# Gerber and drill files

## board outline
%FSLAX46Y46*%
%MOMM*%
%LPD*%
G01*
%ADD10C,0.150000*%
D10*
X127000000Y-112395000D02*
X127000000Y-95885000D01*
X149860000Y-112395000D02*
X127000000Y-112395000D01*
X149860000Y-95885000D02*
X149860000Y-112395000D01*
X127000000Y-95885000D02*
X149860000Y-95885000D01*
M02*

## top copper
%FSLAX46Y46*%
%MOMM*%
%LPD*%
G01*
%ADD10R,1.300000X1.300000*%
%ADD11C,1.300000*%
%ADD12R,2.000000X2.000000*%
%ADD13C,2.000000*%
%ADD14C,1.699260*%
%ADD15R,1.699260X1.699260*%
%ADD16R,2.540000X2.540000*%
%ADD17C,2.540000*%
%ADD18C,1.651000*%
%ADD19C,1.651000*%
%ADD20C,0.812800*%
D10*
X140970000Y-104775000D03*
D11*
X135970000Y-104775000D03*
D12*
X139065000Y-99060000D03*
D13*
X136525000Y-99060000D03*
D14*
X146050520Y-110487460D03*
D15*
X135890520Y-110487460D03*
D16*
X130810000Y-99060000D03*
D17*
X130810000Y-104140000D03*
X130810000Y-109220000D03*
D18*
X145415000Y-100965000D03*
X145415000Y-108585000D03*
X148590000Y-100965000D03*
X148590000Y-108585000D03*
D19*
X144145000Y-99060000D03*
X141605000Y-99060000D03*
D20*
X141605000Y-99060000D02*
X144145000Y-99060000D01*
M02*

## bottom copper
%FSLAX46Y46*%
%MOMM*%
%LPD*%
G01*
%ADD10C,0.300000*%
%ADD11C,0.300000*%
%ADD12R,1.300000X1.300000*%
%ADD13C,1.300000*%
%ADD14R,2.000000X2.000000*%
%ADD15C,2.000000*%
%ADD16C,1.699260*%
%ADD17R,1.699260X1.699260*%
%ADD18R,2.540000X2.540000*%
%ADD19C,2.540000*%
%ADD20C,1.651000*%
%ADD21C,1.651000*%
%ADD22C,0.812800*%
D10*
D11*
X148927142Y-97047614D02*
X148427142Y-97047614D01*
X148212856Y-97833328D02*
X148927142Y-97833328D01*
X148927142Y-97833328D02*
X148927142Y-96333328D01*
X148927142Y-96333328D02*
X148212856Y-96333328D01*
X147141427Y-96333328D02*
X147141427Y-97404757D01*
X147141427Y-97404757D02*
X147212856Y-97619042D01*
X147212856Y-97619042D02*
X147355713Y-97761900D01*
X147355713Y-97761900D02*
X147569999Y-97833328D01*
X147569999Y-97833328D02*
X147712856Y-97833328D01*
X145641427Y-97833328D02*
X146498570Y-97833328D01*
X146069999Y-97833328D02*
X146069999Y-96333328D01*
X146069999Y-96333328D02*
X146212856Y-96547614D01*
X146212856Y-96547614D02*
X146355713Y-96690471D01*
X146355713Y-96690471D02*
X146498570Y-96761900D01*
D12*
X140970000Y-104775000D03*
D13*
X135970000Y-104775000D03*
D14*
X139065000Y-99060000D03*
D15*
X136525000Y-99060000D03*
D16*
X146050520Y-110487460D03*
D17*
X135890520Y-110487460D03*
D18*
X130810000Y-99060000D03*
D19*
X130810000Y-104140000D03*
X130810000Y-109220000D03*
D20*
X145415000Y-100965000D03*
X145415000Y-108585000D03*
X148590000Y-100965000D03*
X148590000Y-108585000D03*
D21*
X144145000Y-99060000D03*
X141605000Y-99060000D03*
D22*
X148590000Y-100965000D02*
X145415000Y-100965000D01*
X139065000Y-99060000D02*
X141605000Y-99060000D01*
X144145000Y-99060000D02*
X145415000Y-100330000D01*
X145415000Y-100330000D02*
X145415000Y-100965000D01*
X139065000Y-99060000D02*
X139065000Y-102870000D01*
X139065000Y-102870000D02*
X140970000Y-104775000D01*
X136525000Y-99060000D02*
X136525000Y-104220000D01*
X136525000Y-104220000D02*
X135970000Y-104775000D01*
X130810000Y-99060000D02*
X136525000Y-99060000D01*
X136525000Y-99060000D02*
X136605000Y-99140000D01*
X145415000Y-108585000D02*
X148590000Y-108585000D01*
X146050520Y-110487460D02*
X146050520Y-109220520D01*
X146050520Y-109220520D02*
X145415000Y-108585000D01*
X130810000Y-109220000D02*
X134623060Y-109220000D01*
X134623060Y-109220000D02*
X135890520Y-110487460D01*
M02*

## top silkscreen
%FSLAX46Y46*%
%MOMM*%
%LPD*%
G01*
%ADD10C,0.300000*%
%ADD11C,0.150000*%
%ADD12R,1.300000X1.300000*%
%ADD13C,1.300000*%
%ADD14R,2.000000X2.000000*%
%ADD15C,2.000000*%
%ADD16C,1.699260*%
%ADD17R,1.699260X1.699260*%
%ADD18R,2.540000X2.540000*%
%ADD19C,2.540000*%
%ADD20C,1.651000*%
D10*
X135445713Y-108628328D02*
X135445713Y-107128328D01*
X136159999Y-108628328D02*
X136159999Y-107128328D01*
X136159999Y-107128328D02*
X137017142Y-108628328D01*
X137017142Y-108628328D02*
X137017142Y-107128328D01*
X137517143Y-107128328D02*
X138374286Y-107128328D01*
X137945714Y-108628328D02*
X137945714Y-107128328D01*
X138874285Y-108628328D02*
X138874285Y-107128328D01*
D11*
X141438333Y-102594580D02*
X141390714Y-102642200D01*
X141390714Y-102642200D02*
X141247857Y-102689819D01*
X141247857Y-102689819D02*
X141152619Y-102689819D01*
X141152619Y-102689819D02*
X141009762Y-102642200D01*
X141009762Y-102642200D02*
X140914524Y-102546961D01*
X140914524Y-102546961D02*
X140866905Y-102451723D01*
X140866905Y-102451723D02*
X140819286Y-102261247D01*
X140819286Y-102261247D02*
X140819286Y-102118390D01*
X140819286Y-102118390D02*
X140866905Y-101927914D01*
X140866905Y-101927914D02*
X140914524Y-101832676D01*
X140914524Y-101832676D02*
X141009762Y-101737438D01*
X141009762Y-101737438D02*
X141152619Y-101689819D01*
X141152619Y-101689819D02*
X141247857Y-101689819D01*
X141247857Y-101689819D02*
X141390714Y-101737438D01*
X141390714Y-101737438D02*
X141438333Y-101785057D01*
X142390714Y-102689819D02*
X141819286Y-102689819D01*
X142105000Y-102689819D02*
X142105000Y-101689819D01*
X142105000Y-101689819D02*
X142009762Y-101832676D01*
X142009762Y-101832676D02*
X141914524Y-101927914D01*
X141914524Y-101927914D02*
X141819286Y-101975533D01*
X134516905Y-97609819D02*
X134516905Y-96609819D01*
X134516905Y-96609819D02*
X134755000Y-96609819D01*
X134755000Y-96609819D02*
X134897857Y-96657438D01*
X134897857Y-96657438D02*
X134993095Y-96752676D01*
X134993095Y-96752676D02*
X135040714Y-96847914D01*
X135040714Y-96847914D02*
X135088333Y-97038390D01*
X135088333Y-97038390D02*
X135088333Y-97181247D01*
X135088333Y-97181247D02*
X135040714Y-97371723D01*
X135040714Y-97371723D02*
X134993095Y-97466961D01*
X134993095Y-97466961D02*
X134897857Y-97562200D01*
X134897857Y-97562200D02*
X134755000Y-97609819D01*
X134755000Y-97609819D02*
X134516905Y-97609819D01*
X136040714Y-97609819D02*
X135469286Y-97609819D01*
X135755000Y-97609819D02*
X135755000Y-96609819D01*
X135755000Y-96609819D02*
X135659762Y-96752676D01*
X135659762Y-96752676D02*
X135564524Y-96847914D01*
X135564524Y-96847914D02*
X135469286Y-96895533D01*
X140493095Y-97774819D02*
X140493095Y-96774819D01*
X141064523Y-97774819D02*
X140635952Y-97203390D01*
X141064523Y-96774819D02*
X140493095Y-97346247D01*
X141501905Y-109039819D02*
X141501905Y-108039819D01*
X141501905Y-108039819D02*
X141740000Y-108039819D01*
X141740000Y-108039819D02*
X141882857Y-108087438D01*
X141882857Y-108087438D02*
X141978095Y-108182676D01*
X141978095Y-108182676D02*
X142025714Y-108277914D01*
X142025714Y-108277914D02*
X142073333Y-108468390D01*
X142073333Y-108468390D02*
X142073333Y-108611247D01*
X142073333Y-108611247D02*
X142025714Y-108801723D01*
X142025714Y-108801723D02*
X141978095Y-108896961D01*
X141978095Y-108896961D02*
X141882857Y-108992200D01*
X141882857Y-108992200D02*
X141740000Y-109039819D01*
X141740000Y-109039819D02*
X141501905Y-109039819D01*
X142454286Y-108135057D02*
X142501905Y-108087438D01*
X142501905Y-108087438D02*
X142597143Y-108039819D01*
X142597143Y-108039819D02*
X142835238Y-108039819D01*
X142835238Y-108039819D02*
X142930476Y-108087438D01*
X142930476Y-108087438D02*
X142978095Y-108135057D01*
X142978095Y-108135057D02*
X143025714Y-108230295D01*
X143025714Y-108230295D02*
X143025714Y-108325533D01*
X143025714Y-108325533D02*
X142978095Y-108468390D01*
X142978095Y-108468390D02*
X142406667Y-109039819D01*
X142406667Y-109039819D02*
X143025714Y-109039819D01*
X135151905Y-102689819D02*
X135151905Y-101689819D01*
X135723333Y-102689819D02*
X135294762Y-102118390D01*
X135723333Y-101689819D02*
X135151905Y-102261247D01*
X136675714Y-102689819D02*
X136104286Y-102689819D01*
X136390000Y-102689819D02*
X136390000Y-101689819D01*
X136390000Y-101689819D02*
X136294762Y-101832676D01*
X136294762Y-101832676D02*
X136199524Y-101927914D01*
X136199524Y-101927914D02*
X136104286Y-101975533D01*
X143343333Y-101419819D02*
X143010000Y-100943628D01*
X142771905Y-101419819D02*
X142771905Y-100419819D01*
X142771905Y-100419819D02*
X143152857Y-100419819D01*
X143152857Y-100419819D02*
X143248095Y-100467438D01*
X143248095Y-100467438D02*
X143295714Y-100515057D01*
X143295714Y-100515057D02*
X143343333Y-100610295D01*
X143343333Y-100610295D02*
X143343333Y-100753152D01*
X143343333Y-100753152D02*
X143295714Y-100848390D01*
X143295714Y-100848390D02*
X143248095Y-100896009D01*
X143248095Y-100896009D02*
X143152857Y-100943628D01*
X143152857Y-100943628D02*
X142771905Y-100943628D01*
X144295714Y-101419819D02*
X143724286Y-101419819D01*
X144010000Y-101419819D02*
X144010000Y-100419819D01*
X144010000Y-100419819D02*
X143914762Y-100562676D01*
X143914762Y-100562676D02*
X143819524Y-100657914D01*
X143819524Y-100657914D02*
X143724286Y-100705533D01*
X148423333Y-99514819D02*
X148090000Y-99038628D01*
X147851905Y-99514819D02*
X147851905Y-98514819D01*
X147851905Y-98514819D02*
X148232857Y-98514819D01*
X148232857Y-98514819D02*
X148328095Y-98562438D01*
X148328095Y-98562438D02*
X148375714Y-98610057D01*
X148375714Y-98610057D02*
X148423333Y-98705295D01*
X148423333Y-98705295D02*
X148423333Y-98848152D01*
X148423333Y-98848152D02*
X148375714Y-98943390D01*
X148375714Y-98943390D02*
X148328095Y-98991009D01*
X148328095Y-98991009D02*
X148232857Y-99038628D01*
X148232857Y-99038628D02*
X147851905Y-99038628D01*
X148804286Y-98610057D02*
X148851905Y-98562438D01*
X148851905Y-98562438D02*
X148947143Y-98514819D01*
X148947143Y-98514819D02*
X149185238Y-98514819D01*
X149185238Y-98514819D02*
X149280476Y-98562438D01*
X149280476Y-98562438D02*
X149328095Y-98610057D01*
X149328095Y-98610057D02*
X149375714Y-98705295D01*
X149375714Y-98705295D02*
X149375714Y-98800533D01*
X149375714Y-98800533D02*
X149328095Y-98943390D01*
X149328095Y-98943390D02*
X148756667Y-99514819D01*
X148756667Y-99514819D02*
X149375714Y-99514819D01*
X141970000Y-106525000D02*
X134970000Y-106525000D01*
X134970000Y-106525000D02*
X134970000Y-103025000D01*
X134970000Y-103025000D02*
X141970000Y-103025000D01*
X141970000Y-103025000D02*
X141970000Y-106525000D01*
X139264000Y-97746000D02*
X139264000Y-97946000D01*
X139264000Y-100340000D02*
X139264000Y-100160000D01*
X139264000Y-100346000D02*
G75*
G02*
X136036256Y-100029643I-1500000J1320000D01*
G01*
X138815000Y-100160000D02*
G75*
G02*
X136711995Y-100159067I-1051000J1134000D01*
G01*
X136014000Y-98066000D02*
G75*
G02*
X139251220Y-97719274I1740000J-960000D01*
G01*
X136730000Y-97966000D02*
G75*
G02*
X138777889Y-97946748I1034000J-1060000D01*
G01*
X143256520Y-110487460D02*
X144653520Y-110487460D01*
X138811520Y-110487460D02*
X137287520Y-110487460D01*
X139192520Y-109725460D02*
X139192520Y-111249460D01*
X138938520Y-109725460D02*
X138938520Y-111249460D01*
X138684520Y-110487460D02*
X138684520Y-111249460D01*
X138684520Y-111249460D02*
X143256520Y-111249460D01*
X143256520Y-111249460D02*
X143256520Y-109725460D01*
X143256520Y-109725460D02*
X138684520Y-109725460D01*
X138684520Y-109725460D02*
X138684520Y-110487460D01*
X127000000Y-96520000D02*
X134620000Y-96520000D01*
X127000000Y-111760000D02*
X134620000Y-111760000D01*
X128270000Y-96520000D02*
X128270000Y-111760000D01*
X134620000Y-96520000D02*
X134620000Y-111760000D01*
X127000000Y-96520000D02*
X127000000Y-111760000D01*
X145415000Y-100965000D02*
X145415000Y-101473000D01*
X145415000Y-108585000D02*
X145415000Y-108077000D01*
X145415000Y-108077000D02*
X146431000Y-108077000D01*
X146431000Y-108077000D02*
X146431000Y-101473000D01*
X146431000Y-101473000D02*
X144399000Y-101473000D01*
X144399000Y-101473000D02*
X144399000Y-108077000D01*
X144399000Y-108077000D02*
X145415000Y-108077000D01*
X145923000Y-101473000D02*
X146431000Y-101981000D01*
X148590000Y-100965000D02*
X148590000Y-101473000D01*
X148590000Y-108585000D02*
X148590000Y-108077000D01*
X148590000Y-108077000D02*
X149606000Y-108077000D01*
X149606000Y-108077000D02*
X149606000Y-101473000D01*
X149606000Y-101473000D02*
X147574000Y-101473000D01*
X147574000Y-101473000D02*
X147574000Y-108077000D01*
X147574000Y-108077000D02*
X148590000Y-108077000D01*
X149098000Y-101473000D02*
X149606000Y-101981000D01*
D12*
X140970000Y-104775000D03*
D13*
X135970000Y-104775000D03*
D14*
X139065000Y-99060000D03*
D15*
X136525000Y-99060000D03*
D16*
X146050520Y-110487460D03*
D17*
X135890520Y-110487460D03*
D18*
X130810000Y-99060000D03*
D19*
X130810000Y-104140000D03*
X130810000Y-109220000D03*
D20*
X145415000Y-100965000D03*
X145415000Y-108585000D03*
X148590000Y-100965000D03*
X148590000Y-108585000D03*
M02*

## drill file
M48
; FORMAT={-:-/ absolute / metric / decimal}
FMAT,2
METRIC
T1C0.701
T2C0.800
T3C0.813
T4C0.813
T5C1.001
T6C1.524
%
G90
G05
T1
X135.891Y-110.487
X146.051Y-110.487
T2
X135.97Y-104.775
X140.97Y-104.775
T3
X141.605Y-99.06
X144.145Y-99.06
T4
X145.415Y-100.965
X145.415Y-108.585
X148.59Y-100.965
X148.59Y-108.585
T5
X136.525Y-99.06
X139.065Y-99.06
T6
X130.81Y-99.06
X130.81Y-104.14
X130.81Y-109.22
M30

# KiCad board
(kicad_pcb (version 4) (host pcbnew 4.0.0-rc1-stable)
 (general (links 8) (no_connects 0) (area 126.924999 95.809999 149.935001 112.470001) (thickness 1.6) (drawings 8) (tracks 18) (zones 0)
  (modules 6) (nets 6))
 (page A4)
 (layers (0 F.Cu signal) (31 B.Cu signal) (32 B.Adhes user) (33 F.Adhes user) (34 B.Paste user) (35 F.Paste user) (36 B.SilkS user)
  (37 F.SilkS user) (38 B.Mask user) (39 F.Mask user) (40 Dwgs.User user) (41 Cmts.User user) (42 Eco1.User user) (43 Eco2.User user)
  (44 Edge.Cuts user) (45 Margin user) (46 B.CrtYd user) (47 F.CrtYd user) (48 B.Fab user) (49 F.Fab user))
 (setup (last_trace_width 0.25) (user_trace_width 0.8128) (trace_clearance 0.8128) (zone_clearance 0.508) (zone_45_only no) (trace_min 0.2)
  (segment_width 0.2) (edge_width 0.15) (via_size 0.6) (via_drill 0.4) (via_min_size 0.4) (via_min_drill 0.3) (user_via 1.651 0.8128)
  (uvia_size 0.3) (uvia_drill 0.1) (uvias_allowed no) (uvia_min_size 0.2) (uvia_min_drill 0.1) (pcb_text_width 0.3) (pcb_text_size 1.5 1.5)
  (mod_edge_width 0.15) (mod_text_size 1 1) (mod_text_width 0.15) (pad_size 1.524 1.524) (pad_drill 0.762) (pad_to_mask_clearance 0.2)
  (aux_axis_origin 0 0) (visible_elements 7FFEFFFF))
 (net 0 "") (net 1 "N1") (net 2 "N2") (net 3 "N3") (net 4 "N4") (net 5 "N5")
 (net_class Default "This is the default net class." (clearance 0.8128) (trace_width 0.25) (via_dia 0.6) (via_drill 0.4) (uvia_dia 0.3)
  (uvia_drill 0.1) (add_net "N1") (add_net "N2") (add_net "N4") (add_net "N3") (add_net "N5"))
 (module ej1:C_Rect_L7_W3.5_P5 (layer F.Cu) (at 140.97 104.775 180)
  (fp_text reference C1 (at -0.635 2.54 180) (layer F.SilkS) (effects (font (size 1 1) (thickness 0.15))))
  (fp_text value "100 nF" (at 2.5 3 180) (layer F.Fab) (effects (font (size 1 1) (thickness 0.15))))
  (fp_line (start -1 -1.75) (end 6 -1.75) (layer F.SilkS) (width 0.15))
  (fp_line (start 6 -1.75) (end 6 1.75) (layer F.SilkS) (width 0.15))
  (fp_line (start 6 1.75) (end -1 1.75) (layer F.SilkS) (width 0.15))
  (fp_line (start -1 1.75) (end -1 -1.75) (layer F.SilkS) (width 0.15))
  (pad 1 thru_hole rect (at 0 0 180) (size 1.3 1.3) (drill 0.8) (layers *.Cu *.Mask F.SilkS) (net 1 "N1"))
  (pad 2 thru_hole circle (at 5 0 180) (size 1.3 1.3) (drill 0.8) (layers *.Cu *.Mask F.SilkS) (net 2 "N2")))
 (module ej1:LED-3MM (layer F.Cu) (at 139.065 99.06 180)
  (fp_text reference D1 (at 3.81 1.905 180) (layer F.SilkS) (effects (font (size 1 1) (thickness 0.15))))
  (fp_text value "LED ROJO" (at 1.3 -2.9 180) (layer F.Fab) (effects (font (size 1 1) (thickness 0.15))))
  (fp_line (start -0.199 1.314) (end -0.199 1.114) (layer F.SilkS) (width 0.15))
  (fp_line (start -0.199 -1.28) (end -0.199 -1.1) (layer F.SilkS) (width 0.15))
  (fp_arc (start 1.301 0.034) (end -0.199 -1.286) (angle 108.5) (layer F.SilkS) (width 0.15))
  (fp_arc (start 1.301 0.034) (end 0.25 -1.1) (angle 85.7) (layer F.SilkS) (width 0.15))
  (fp_arc (start 1.311 0.034) (end 3.051 0.994) (angle 110) (layer F.SilkS) (width 0.15))
  (fp_arc (start 1.301 0.034) (end 2.335 1.094) (angle 87.5) (layer F.SilkS) (width 0.15))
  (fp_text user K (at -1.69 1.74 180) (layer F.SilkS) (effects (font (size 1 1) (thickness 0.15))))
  (pad 1 thru_hole rect (at 0 0 270) (size 2 2) (drill 1.00076) (layers *.Cu *.Mask F.SilkS) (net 1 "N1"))
  (pad 2 thru_hole circle (at 2.54 0 180) (size 2 2) (drill 1.00076) (layers *.Cu *.Mask F.SilkS) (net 2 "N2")))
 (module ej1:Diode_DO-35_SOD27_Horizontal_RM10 (layer F.Cu) (at 135.89 110.49)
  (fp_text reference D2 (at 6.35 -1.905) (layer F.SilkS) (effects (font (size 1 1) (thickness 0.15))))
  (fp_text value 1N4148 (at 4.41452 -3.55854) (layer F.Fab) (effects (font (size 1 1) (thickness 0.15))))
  (fp_line (start 7.36652 -0.00254) (end 8.76352 -0.00254) (layer F.SilkS) (width 0.15))
  (fp_line (start 2.92152 -0.00254) (end 1.39752 -0.00254) (layer F.SilkS) (width 0.15))
  (fp_line (start 3.30252 -0.76454) (end 3.30252 0.75946) (layer F.SilkS) (width 0.15))
  (fp_line (start 3.04852 -0.76454) (end 3.04852 0.75946) (layer F.SilkS) (width 0.15))
  (fp_line (start 2.79452 -0.00254) (end 2.79452 0.75946) (layer F.SilkS) (width 0.15))
  (fp_line (start 2.79452 0.75946) (end 7.36652 0.75946) (layer F.SilkS) (width 0.15))
  (fp_line (start 7.36652 0.75946) (end 7.36652 -0.76454) (layer F.SilkS) (width 0.15))
  (fp_line (start 7.36652 -0.76454) (end 2.79452 -0.76454) (layer F.SilkS) (width 0.15))
  (fp_line (start 2.79452 -0.76454) (end 2.79452 -0.00254) (layer F.SilkS) (width 0.15))
  (pad 2 thru_hole circle (at 10.16052 -0.00254 180) (size 1.69926 1.69926) (drill 0.70104) (layers *.Cu *.Mask F.SilkS) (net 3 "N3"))
  (pad 1 thru_hole rect (at 0.00052 -0.00254 180) (size 1.69926 1.69926) (drill 0.70104) (layers *.Cu *.Mask F.SilkS) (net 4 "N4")))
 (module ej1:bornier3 (layer F.Cu) (at 130.81 104.14 270)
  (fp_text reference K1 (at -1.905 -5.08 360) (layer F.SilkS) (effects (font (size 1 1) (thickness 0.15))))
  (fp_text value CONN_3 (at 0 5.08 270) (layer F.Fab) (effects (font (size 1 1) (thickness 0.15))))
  (fp_line (start -7.62 3.81) (end -7.62 -3.81) (layer F.SilkS) (width 0.15))
  (fp_line (start 7.62 3.81) (end 7.62 -3.81) (layer F.SilkS) (width 0.15))
  (fp_line (start -7.62 2.54) (end 7.62 2.54) (layer F.SilkS) (width 0.15))
  (fp_line (start -7.62 -3.81) (end 7.62 -3.81) (layer F.SilkS) (width 0.15))
  (fp_line (start -7.62 3.81) (end 7.62 3.81) (layer F.SilkS) (width 0.15))
  (pad 1 thru_hole rect (at -5.08 0 270) (size 2.54 2.54) (drill 1.524) (layers *.Cu *.Mask F.SilkS) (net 2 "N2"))
  (pad 2 thru_hole circle (at 0 0 270) (size 2.54 2.54) (drill 1.524) (layers *.Cu *.Mask F.SilkS) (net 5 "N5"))
  (pad 3 thru_hole circle (at 5.08 0 270) (size 2.54 2.54) (drill 1.524) (layers *.Cu *.Mask F.SilkS) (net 4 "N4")))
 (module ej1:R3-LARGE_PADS (layer F.Cu) (at 145.415 104.775 270)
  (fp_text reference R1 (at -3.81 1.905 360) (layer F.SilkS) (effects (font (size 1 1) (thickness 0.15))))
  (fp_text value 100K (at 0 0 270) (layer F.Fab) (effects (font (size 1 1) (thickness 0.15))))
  (fp_line (start -3.81 0) (end -3.302 0) (layer F.SilkS) (width 0.15))
  (fp_line (start 3.81 0) (end 3.302 0) (layer F.SilkS) (width 0.15))
  (fp_line (start 3.302 0) (end 3.302 -1.016) (layer F.SilkS) (width 0.15))
  (fp_line (start 3.302 -1.016) (end -3.302 -1.016) (layer F.SilkS) (width 0.15))
  (fp_line (start -3.302 -1.016) (end -3.302 1.016) (layer F.SilkS) (width 0.15))
  (fp_line (start -3.302 1.016) (end 3.302 1.016) (layer F.SilkS) (width 0.15))
  (fp_line (start 3.302 1.016) (end 3.302 0) (layer F.SilkS) (width 0.15))
  (fp_line (start -3.302 -0.508) (end -2.794 -1.016) (layer F.SilkS) (width 0.15))
  (pad 1 thru_hole circle (at -3.81 0 270) (size 1.651 1.651) (drill 0.8128) (layers *.Cu *.Mask F.SilkS) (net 1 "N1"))
  (pad 2 thru_hole circle (at 3.81 0 270) (size 1.651 1.651) (drill 0.8128) (layers *.Cu *.Mask F.SilkS) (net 3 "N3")))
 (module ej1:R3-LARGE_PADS (layer F.Cu) (at 148.59 104.775 270)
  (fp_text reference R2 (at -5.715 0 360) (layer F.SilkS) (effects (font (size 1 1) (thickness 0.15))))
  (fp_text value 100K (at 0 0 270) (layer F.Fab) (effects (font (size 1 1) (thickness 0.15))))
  (fp_line (start -3.81 0) (end -3.302 0) (layer F.SilkS) (width 0.15))
  (fp_line (start 3.81 0) (end 3.302 0) (layer F.SilkS) (width 0.15))
  (fp_line (start 3.302 0) (end 3.302 -1.016) (layer F.SilkS) (width 0.15))
  (fp_line (start 3.302 -1.016) (end -3.302 -1.016) (layer F.SilkS) (width 0.15))
  (fp_line (start -3.302 -1.016) (end -3.302 1.016) (layer F.SilkS) (width 0.15))
  (fp_line (start -3.302 1.016) (end 3.302 1.016) (layer F.SilkS) (width 0.15))
  (fp_line (start 3.302 1.016) (end 3.302 0) (layer F.SilkS) (width 0.15))
  (fp_line (start -3.302 -0.508) (end -2.794 -1.016) (layer F.SilkS) (width 0.15))
  (pad 1 thru_hole circle (at -3.81 0 270) (size 1.651 1.651) (drill 0.8128) (layers *.Cu *.Mask F.SilkS) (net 1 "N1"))
  (pad 2 thru_hole circle (at 3.81 0 270) (size 1.651 1.651) (drill 0.8128) (layers *.Cu *.Mask F.SilkS) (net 3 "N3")))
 (gr_line (start 127 112.395) (end 127 95.885) (angle 90) (layer Edge.Cuts) (width 0.15))
 (gr_line (start 149.86 112.395) (end 127 112.395) (angle 90) (layer Edge.Cuts) (width 0.15))
 (gr_line (start 149.86 95.885) (end 149.86 112.395) (angle 90) (layer Edge.Cuts) (width 0.15))
 (gr_line (start 127 95.885) (end 149.86 95.885) (angle 90) (layer Edge.Cuts) (width 0.15))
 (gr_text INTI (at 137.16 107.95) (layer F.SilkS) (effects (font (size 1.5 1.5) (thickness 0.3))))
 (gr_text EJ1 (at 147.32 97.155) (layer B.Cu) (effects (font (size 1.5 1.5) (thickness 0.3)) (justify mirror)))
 (segment (start 148.59 100.965) (end 145.415 100.965) (width 0.8128) (layer B.Cu) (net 1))
 (segment (start 139.065 99.06) (end 141.605 99.06) (width 0.8128) (layer B.Cu) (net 1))
 (segment (start 144.145 99.06) (end 145.415 100.33) (width 0.8128) (layer B.Cu) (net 1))
 (via (at 144.145 99.06) (size 1.651) (drill 0.8128) (layers F.Cu B.Cu) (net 1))
 (segment (start 141.605 99.06) (end 144.145 99.06) (width 0.8128) (layer F.Cu) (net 1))
 (via (at 141.605 99.06) (size 1.651) (drill 0.8128) (layers F.Cu B.Cu) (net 1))
 (segment (start 145.415 100.33) (end 145.415 100.965) (width 0.8128) (layer B.Cu) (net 1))
 (segment (start 139.065 99.06) (end 139.065 102.87) (width 0.8128) (layer B.Cu) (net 1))
 (segment (start 139.065 102.87) (end 140.97 104.775) (width 0.8128) (layer B.Cu) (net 1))
 (segment (start 136.525 99.06) (end 136.525 104.22) (width 0.8128) (layer B.Cu) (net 2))
 (segment (start 136.525 104.22) (end 135.97 104.775) (width 0.8128) (layer B.Cu) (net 2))
 (segment (start 130.81 99.06) (end 136.525 99.06) (width 0.8128) (layer B.Cu) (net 2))
 (segment (start 136.525 99.06) (end 136.605 99.14) (width 0.8128) (layer B.Cu) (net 2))
 (segment (start 145.415 108.585) (end 148.59 108.585) (width 0.8128) (layer B.Cu) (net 3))
 (segment (start 146.05052 110.48746) (end 146.05052 109.22052) (width 0.8128) (layer B.Cu) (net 3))
 (segment (start 146.05052 109.22052) (end 145.415 108.585) (width 0.8128) (layer B.Cu) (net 3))
 (segment (start 130.81 109.22) (end 134.62306 109.22) (width 0.8128) (layer B.Cu) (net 4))
 (segment (start 134.62306 109.22) (end 135.89052 110.48746) (width 0.8128) (layer B.Cu) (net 4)))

